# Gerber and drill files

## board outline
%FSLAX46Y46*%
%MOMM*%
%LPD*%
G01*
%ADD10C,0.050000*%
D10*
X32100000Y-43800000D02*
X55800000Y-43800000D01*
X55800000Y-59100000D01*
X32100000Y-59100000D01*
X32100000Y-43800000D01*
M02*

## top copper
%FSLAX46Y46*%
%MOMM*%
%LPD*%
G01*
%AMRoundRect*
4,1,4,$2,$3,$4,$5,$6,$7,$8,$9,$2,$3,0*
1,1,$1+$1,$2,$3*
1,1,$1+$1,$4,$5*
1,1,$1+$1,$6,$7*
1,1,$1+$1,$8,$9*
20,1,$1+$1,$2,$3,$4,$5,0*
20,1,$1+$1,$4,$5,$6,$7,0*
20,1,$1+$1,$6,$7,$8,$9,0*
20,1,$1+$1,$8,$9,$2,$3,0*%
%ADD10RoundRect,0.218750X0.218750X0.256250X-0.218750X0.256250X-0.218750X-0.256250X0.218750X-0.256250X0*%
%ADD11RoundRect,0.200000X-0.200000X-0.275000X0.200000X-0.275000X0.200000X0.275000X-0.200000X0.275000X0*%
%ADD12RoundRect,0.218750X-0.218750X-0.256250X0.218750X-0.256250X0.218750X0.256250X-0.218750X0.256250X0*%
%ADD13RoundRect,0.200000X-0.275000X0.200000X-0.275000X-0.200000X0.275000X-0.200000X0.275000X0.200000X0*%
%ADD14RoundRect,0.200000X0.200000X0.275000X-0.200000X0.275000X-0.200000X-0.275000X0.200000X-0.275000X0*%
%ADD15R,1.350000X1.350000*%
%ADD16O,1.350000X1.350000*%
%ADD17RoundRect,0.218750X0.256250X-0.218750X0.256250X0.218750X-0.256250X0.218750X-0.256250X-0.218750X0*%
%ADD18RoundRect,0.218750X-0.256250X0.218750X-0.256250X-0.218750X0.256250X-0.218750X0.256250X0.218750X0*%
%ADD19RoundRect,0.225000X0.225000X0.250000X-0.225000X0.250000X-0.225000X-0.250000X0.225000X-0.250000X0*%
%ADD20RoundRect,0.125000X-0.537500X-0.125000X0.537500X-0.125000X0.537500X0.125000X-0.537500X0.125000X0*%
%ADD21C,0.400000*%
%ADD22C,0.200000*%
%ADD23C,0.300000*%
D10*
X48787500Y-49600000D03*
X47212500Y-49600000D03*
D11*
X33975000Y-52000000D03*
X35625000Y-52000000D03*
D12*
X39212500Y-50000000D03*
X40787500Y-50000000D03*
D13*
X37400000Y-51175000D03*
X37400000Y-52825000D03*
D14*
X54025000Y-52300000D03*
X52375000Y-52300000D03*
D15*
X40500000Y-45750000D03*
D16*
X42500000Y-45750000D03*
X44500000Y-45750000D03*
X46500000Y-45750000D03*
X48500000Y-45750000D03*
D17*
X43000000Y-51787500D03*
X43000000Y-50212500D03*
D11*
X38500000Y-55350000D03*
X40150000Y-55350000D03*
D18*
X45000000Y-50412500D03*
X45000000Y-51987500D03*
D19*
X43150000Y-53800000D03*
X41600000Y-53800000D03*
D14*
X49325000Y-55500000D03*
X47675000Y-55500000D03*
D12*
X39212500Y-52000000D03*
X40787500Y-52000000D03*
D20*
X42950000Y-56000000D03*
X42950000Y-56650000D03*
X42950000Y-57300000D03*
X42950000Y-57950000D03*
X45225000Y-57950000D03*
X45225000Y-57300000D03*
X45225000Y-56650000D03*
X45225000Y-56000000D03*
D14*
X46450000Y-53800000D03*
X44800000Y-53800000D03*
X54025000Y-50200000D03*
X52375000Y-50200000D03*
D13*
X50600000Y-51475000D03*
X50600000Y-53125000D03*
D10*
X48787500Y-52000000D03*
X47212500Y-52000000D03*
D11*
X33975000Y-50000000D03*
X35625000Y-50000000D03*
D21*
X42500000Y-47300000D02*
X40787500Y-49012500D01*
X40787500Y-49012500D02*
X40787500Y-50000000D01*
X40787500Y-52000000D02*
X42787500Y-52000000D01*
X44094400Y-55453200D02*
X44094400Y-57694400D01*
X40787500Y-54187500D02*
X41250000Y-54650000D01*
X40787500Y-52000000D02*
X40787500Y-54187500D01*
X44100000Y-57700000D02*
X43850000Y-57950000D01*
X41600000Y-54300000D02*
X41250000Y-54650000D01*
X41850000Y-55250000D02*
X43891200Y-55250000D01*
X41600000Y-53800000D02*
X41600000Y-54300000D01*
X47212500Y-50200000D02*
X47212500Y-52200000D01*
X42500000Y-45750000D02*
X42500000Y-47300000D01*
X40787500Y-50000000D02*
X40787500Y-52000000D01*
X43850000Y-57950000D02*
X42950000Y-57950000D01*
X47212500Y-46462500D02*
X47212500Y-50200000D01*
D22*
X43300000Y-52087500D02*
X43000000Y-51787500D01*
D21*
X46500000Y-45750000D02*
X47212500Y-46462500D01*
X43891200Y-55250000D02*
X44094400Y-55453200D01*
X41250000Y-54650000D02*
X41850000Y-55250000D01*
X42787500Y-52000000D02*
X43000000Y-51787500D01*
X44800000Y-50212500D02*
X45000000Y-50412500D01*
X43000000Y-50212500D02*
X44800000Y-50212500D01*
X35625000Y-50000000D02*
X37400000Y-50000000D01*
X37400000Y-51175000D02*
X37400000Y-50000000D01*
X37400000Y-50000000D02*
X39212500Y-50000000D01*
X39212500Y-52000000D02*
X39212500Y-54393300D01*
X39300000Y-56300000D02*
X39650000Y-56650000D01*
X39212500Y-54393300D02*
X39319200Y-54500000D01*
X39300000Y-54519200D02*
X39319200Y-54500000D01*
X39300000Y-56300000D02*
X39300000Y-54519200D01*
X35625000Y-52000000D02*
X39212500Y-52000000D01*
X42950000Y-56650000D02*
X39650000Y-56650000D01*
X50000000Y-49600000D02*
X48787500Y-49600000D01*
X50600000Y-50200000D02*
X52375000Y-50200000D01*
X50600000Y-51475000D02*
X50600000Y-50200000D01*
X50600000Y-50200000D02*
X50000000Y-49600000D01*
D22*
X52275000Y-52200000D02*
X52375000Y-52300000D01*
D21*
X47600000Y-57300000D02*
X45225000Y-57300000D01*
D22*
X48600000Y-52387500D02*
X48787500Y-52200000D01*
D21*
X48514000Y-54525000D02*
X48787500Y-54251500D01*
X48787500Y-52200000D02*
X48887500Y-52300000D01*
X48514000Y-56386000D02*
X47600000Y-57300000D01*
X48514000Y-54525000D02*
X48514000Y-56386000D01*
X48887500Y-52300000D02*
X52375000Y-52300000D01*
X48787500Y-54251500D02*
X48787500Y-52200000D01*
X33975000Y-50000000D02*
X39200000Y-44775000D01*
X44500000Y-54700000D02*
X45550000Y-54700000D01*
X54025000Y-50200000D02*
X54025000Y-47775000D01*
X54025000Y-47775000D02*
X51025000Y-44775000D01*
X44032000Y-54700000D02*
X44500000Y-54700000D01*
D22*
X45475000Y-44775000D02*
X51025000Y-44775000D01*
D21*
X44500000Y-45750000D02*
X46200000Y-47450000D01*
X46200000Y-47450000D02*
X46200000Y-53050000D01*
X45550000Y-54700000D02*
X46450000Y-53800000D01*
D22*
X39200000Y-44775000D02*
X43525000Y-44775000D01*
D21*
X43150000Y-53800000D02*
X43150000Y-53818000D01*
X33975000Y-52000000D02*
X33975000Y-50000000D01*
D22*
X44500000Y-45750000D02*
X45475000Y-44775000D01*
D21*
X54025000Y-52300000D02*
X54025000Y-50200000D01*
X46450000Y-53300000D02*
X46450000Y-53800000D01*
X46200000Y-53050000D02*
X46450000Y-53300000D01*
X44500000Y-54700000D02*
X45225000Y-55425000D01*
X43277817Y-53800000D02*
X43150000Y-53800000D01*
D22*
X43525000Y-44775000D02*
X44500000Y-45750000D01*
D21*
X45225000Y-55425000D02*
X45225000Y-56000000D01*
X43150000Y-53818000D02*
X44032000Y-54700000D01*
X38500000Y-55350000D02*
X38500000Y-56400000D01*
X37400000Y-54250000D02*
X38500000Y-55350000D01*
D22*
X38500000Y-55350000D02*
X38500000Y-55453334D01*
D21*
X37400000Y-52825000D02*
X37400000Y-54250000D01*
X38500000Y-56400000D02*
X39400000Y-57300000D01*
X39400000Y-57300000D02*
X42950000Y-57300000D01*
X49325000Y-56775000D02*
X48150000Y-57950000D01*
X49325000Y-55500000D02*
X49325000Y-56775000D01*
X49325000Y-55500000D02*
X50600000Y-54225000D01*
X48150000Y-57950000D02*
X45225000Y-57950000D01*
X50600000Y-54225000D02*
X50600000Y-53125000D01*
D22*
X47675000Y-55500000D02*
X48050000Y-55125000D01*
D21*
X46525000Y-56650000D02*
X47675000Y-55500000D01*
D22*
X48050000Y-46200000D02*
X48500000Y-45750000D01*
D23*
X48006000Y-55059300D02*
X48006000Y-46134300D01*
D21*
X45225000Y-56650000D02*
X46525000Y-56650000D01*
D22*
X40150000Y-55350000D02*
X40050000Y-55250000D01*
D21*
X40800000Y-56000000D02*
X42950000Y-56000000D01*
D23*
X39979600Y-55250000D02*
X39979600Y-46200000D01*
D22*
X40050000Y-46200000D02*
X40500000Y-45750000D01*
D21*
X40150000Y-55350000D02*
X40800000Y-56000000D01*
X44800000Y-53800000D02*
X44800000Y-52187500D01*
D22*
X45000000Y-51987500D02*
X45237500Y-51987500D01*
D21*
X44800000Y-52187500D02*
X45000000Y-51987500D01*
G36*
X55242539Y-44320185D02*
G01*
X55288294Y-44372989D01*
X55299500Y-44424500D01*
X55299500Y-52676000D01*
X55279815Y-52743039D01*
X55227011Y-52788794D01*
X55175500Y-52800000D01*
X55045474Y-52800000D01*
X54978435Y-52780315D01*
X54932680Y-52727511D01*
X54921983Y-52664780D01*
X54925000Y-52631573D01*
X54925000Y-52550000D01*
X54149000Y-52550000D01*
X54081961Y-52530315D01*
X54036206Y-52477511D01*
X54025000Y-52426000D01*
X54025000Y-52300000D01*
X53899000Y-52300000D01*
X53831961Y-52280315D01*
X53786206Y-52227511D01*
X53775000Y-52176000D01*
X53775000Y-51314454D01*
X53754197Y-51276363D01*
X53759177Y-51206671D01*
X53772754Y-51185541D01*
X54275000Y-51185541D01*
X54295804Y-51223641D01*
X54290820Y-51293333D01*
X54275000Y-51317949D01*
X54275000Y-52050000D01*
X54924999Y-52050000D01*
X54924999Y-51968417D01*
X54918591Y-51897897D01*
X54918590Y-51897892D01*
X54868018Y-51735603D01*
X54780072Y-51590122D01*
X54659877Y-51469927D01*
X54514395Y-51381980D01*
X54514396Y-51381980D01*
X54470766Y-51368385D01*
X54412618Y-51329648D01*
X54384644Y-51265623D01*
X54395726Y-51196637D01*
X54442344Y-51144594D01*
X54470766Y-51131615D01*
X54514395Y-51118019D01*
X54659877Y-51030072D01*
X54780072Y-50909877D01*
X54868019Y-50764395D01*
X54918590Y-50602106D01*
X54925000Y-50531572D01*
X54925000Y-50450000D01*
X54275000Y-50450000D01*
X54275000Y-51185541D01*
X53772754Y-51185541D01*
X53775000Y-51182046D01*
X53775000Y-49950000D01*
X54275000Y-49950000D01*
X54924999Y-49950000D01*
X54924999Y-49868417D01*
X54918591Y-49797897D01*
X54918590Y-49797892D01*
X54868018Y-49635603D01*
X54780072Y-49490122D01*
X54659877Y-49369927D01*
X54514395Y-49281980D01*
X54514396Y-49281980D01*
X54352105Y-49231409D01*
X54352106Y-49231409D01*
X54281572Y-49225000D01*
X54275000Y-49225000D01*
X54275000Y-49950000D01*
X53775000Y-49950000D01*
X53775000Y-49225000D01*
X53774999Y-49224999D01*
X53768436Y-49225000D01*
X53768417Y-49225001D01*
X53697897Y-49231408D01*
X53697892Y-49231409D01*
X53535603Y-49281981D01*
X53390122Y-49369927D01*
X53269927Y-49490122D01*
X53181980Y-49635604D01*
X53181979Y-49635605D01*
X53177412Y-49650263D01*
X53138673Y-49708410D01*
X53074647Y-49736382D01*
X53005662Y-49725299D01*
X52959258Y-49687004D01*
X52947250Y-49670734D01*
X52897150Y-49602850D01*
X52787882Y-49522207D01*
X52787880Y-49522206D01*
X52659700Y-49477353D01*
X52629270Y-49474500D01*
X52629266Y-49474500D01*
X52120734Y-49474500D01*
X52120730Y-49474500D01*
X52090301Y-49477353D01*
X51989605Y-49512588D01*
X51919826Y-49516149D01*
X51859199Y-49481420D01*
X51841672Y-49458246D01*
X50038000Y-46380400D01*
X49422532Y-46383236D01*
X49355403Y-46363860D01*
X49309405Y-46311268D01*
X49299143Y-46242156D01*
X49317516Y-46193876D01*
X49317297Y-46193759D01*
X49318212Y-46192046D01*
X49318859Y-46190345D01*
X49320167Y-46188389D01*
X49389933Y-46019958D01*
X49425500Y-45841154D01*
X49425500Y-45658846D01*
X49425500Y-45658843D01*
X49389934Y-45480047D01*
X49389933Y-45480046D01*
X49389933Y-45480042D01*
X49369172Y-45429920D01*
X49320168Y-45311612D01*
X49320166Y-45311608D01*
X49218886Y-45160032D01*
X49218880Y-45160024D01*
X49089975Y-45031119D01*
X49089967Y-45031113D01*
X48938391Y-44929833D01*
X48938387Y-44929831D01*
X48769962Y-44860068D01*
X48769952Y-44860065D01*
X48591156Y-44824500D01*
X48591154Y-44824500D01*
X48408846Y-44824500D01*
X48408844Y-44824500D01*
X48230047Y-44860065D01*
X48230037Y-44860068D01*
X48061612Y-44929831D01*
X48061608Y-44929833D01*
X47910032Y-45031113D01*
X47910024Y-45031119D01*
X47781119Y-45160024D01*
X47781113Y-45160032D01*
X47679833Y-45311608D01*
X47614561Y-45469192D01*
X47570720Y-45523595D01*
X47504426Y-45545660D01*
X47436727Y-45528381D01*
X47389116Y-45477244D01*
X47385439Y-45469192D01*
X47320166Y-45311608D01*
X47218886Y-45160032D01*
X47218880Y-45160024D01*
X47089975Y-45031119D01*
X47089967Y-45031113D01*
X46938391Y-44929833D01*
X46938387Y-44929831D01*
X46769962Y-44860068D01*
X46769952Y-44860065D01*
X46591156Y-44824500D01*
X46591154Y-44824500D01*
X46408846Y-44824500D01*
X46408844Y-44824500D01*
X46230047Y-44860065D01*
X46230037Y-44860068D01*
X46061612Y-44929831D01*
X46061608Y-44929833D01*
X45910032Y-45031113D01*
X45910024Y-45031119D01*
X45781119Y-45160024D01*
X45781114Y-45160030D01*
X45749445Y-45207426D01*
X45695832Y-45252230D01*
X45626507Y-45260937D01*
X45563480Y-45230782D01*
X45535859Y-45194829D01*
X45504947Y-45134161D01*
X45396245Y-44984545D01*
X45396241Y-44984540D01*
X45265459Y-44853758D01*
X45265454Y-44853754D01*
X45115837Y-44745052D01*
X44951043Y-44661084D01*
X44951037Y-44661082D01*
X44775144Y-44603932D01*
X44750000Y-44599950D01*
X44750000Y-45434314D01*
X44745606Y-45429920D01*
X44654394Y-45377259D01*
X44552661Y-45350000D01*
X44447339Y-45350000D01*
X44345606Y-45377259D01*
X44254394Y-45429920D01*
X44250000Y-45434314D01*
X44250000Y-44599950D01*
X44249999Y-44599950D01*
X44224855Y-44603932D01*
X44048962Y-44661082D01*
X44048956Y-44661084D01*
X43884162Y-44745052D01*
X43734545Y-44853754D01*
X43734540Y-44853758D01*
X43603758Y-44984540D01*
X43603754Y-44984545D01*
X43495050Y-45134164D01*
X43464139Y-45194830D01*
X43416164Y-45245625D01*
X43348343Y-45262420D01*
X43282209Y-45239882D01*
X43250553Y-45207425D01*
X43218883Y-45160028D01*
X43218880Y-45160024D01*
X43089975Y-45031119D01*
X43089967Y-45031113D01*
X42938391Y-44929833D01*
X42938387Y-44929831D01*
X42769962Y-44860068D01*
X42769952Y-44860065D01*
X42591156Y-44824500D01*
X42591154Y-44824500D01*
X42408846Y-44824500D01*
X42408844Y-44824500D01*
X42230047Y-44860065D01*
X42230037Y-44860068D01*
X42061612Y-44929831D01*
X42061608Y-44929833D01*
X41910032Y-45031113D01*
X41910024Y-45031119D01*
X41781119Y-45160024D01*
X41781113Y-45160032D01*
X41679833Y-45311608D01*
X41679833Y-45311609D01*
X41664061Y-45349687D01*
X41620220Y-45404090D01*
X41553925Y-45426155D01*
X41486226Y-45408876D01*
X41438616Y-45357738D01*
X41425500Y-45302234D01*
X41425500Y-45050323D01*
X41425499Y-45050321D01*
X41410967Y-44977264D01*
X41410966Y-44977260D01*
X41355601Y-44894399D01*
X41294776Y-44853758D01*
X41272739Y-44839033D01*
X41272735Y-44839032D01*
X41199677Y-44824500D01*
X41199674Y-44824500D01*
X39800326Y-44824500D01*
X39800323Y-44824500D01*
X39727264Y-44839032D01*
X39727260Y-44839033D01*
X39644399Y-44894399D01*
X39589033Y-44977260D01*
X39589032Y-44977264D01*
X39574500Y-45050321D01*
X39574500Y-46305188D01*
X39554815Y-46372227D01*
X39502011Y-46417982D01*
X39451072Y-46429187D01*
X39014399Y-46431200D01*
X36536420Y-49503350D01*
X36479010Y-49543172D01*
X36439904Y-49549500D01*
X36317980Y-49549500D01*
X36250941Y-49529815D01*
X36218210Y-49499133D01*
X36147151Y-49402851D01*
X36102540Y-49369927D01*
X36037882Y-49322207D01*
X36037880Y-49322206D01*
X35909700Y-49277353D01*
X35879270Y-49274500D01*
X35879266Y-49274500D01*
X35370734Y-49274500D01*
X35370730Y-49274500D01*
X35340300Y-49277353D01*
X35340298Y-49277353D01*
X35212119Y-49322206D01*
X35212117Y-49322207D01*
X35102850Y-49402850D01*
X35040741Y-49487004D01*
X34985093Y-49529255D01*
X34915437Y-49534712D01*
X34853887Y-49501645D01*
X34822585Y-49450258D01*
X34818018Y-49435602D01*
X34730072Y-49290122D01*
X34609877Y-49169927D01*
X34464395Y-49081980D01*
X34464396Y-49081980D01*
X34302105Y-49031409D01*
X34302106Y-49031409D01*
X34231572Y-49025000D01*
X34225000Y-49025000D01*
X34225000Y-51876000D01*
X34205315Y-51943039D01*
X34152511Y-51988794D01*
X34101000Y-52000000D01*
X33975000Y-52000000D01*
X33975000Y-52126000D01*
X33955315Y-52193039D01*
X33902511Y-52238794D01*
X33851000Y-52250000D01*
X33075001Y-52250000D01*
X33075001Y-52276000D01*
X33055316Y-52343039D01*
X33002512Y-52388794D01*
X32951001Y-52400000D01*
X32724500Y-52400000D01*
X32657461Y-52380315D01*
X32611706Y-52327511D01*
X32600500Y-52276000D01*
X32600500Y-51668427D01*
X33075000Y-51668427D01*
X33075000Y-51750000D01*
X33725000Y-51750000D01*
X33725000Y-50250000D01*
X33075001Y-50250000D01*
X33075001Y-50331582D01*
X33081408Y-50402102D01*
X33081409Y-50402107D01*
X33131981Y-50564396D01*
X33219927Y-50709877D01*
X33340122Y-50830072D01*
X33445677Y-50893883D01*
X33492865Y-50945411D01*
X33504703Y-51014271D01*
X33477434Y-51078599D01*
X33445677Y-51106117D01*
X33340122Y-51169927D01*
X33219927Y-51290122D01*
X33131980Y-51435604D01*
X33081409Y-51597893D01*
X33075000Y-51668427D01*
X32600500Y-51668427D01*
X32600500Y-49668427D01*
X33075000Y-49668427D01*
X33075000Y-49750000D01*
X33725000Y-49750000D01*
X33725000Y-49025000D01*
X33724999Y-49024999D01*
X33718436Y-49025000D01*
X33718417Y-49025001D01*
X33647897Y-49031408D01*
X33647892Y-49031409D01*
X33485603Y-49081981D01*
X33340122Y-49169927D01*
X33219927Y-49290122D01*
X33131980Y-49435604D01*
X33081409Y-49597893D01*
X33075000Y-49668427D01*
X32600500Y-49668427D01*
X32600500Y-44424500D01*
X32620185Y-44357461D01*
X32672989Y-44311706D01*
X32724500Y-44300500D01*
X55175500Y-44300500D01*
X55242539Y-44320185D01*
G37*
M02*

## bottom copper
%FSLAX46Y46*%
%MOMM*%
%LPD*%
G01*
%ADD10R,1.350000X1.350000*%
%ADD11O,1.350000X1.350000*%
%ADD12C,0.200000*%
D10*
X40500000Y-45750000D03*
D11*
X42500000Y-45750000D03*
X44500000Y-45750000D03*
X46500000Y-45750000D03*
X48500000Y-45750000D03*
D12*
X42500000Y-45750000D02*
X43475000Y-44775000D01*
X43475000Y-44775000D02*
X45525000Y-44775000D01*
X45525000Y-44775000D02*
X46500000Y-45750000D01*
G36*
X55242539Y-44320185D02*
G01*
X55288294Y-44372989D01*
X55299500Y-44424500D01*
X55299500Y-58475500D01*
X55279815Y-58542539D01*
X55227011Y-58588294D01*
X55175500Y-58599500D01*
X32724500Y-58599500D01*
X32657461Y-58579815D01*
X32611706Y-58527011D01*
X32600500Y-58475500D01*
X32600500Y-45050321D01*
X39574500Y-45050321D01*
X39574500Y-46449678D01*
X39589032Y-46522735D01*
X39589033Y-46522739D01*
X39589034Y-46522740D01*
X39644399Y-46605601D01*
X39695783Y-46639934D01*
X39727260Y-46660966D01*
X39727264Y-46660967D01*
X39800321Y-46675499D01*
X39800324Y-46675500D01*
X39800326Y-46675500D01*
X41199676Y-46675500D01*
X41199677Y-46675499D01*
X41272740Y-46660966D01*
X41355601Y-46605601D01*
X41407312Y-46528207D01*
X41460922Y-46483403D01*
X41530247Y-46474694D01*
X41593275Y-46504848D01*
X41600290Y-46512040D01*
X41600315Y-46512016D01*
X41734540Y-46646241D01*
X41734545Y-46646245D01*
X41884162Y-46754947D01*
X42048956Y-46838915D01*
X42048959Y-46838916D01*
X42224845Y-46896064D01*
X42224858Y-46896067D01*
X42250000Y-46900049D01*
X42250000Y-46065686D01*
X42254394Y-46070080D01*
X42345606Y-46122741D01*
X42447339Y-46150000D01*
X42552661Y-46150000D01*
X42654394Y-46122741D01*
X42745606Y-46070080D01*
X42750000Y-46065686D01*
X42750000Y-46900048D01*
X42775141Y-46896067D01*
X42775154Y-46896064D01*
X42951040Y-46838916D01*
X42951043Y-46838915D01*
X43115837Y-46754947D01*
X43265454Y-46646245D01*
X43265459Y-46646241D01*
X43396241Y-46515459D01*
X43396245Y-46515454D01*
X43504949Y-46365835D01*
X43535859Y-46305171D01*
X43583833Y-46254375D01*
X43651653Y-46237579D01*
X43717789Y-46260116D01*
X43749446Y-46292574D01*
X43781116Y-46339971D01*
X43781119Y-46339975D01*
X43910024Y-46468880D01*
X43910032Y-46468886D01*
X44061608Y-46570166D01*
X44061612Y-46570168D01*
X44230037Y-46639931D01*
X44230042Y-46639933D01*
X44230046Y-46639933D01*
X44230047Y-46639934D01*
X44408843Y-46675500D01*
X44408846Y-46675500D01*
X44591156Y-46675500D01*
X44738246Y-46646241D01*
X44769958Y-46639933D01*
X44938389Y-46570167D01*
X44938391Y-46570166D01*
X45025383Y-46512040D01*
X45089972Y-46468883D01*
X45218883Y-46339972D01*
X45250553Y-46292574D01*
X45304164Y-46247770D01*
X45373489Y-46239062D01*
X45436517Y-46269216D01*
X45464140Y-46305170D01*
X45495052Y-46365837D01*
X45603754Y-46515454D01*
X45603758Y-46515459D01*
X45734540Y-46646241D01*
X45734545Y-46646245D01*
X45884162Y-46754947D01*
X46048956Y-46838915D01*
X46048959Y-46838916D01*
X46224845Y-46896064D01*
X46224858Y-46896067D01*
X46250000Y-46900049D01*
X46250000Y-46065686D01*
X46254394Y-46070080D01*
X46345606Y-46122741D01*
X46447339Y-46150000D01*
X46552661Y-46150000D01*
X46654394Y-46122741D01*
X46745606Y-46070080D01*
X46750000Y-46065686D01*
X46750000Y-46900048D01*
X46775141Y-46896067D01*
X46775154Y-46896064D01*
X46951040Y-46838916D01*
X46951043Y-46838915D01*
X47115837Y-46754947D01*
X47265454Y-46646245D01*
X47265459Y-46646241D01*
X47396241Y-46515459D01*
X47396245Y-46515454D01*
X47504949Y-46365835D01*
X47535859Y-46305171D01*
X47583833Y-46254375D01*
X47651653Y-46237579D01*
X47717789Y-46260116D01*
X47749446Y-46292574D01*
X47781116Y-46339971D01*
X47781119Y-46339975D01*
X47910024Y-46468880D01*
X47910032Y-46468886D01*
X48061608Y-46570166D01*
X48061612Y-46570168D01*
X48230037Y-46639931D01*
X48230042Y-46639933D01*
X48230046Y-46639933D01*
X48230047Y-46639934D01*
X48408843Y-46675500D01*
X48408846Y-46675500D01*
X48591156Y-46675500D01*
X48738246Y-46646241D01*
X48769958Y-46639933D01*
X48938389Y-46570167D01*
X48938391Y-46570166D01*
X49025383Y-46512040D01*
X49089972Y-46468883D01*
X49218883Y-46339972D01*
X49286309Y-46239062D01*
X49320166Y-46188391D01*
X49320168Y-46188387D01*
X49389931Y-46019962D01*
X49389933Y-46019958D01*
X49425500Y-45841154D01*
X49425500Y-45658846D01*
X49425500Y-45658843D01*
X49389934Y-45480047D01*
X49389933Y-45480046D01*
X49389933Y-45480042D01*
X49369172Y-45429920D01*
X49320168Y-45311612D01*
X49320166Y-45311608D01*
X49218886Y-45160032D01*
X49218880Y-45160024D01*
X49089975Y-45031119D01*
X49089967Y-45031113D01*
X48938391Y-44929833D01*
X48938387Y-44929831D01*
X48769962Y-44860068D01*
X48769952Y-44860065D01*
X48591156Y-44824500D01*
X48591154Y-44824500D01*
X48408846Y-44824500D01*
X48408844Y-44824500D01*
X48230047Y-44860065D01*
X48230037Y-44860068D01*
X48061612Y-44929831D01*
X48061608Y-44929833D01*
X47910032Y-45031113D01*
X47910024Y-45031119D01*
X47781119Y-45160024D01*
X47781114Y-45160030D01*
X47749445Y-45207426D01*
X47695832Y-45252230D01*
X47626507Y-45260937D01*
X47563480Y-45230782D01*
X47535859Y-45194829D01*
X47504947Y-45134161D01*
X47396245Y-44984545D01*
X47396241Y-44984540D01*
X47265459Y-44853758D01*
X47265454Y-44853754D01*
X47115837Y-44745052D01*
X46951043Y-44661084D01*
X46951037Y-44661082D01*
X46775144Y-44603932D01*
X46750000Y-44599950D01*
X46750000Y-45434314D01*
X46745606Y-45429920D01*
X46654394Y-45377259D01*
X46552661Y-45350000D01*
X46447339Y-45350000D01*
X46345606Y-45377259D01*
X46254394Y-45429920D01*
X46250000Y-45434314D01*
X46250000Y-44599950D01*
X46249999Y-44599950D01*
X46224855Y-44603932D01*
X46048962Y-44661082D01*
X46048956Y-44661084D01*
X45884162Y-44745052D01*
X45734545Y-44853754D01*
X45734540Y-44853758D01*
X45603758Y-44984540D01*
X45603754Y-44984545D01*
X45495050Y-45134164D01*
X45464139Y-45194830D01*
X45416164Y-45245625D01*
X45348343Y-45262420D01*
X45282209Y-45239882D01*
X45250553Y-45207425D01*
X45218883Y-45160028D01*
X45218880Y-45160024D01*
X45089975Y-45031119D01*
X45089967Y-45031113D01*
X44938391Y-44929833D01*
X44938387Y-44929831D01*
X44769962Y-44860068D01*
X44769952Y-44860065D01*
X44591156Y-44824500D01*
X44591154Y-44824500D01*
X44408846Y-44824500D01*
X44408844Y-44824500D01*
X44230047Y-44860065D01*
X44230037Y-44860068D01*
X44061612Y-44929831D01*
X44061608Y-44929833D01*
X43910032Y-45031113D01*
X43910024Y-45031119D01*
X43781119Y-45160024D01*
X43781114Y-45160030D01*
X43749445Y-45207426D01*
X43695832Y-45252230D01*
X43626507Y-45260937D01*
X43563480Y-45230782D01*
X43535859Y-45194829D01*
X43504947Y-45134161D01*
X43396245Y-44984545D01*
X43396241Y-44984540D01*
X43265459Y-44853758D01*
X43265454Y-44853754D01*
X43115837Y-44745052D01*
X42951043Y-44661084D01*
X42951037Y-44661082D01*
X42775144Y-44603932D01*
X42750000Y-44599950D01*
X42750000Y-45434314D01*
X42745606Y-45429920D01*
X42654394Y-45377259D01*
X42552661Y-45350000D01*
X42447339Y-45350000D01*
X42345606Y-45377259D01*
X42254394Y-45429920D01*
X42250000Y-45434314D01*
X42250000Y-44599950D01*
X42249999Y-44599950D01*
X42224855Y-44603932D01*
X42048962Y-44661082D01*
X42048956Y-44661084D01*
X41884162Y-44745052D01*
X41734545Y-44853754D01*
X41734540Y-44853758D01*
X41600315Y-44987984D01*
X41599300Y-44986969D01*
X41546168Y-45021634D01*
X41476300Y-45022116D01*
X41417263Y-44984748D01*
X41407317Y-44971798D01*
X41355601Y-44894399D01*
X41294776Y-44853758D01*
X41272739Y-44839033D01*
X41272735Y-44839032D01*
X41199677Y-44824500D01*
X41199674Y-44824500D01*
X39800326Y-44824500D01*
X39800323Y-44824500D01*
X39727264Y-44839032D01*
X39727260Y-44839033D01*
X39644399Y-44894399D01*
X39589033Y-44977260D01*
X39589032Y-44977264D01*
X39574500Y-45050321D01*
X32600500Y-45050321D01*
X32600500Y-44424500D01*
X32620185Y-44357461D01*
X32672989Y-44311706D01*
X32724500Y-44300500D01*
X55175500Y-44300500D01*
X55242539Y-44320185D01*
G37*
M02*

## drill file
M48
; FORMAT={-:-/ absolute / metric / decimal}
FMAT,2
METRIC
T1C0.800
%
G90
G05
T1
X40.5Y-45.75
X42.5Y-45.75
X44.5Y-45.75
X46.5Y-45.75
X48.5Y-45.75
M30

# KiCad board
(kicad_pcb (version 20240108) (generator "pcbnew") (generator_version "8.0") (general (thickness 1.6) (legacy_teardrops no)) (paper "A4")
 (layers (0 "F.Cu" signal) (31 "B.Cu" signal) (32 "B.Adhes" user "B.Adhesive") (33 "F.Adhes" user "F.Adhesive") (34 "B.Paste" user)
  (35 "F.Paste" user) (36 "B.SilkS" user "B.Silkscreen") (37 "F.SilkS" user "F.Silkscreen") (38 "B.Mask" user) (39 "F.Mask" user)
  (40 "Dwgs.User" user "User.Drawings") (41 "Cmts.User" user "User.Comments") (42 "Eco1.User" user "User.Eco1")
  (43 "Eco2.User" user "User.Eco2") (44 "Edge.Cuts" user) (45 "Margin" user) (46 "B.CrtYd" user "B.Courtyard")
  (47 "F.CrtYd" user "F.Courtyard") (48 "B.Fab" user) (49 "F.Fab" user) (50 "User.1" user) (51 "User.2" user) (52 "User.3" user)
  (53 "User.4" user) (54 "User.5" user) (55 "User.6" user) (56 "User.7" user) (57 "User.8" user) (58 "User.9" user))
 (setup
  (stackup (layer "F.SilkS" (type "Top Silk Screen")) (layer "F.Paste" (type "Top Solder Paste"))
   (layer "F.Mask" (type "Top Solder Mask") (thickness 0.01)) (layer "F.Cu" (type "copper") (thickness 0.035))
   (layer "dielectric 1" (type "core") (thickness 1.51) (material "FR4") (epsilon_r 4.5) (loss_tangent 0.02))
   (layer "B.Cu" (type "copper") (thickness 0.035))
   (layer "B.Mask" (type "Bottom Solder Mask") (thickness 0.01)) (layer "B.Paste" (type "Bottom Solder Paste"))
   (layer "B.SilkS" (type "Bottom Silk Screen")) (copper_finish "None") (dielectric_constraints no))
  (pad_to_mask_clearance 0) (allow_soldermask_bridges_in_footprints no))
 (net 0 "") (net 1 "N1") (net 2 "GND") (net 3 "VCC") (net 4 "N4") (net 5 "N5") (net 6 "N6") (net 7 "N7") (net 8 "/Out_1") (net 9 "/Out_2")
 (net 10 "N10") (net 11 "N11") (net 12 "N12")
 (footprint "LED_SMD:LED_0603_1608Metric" (layer "F.Cu") (at 48 49.6 180)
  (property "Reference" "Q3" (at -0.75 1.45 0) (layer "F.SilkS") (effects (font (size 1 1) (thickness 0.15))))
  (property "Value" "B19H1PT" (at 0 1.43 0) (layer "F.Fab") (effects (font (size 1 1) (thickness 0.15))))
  (pad "1" smd roundrect (at -0.7875 0 180) (size 0.875 0.95) (layers "F.Cu" "F.Paste" "F.Mask") (roundrect_rratio 0.25) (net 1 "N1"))
  (pad "2" smd roundrect (at 0.7875 0 180) (size 0.875 0.95) (layers "F.Cu" "F.Paste" "F.Mask") (roundrect_rratio 0.25) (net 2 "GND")))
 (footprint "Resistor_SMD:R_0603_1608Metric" (layer "F.Cu") (at 34.8 52)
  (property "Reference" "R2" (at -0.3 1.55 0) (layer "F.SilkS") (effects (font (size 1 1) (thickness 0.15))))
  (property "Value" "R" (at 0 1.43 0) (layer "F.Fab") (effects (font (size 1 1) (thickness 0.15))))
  (pad "1" smd roundrect (at -0.825 0) (size 0.8 0.95) (layers "F.Cu" "F.Paste" "F.Mask") (roundrect_rratio 0.25) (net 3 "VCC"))
  (pad "2" smd roundrect (at 0.825 0) (size 0.8 0.95) (layers "F.Cu" "F.Paste" "F.Mask") (roundrect_rratio 0.25) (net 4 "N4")))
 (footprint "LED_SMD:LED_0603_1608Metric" (layer "F.Cu") (at 40 50)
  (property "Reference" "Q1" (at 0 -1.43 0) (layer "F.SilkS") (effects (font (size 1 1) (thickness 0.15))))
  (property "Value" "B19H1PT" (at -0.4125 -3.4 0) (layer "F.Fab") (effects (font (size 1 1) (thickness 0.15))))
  (pad "1" smd roundrect (at -0.7875 0) (size 0.875 0.95) (layers "F.Cu" "F.Paste" "F.Mask") (roundrect_rratio 0.25) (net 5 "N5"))
  (pad "2" smd roundrect (at 0.7875 0) (size 0.875 0.95) (layers "F.Cu" "F.Paste" "F.Mask") (roundrect_rratio 0.25) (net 2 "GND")))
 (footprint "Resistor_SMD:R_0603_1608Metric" (layer "F.Cu") (at 37.4 52 -90)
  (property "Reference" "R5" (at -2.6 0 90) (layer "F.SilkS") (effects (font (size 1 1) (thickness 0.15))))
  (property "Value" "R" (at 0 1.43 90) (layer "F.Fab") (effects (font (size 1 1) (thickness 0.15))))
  (pad "1" smd roundrect (at -0.825 0 270) (size 0.8 0.95) (layers "F.Cu" "F.Paste" "F.Mask") (roundrect_rratio 0.25) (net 5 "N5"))
  (pad "2" smd roundrect (at 0.825 0 270) (size 0.8 0.95) (layers "F.Cu" "F.Paste" "F.Mask") (roundrect_rratio 0.25) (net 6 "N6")))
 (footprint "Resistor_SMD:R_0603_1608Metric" (layer "F.Cu") (at 53.2 52.3 180)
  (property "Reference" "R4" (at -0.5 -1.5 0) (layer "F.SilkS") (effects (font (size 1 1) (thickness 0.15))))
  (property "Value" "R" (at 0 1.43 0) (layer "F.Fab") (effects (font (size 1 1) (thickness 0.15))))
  (pad "1" smd roundrect (at -0.825 0 180) (size 0.8 0.95) (layers "F.Cu" "F.Paste" "F.Mask") (roundrect_rratio 0.25) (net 3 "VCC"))
  (pad "2" smd roundrect (at 0.825 0 180) (size 0.8 0.95) (layers "F.Cu" "F.Paste" "F.Mask") (roundrect_rratio 0.25) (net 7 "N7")))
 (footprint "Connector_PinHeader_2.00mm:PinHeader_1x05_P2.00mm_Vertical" (layer "F.Cu") (at 40.5 45.75 90)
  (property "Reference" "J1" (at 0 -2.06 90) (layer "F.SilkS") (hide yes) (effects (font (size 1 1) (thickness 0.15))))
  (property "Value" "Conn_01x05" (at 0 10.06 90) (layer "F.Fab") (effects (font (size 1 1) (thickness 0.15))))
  (pad "1" thru_hole rect (at 0 0 90) (size 1.35 1.35) (drill 0.8) (layers "*.Cu" "*.Mask") (remove_unused_layers no) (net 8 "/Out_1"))
  (pad "2" thru_hole oval (at 0 2 90) (size 1.35 1.35) (drill 0.8) (layers "*.Cu" "*.Mask") (remove_unused_layers no) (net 2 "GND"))
  (pad "3" thru_hole oval (at 0 4 90) (size 1.35 1.35) (drill 0.8) (layers "*.Cu" "*.Mask") (remove_unused_layers no) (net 3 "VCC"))
  (pad "4" thru_hole oval (at 0 6 90) (size 1.35 1.35) (drill 0.8) (layers "*.Cu" "*.Mask") (remove_unused_layers no) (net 2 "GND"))
  (pad "5" thru_hole oval (at 0 8 90) (size 1.35 1.35) (drill 0.8) (layers "*.Cu" "*.Mask") (remove_unused_layers no) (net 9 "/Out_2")))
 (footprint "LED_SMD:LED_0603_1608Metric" (layer "F.Cu") (at 43 51 90)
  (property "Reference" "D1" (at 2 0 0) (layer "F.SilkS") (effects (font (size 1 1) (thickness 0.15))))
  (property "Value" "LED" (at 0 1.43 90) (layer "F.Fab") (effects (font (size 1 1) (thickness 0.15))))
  (pad "1" smd roundrect (at -0.7875 0 90) (size 0.875 0.95) (layers "F.Cu" "F.Paste" "F.Mask") (roundrect_rratio 0.25) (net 2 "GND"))
  (pad "2" smd roundrect (at 0.7875 0 90) (size 0.875 0.95) (layers "F.Cu" "F.Paste" "F.Mask") (roundrect_rratio 0.25) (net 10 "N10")))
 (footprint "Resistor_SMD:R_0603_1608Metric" (layer "F.Cu") (at 39.325 55.35)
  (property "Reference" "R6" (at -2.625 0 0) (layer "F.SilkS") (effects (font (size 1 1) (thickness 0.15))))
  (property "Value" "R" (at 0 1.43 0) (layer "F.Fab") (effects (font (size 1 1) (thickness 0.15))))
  (pad "1" smd roundrect (at -0.825 0) (size 0.8 0.95) (layers "F.Cu" "F.Paste" "F.Mask") (roundrect_rratio 0.25) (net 6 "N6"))
  (pad "2" smd roundrect (at 0.825 0) (size 0.8 0.95) (layers "F.Cu" "F.Paste" "F.Mask") (roundrect_rratio 0.25) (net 8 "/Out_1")))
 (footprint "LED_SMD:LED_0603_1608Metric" (layer "F.Cu") (at 45 51.2 -90)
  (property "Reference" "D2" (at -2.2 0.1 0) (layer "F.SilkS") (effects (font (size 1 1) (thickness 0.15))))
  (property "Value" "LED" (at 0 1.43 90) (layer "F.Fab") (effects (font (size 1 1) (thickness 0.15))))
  (pad "1" smd roundrect (at -0.7875 0 270) (size 0.875 0.95) (layers "F.Cu" "F.Paste" "F.Mask") (roundrect_rratio 0.25) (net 10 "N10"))
  (pad "2" smd roundrect (at 0.7875 0 270) (size 0.875 0.95) (layers "F.Cu" "F.Paste" "F.Mask") (roundrect_rratio 0.25) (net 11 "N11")))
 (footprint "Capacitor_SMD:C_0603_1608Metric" (layer "F.Cu") (at 42.375 53.8 180)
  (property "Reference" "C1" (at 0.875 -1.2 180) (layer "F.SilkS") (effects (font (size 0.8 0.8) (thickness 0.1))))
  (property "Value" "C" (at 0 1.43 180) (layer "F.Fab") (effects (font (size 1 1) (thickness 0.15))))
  (pad "1" smd roundrect (at -0.775 0 180) (size 0.9 0.95) (layers "F.Cu" "F.Paste" "F.Mask") (roundrect_rratio 0.25) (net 3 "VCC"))
  (pad "2" smd roundrect (at 0.775 0 180) (size 0.9 0.95) (layers "F.Cu" "F.Paste" "F.Mask") (roundrect_rratio 0.25) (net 2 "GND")))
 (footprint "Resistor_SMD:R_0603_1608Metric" (layer "F.Cu") (at 48.5 55.5 180)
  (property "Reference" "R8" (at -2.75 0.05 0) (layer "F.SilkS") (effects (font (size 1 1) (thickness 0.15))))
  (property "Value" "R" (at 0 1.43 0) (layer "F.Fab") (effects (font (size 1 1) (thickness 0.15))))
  (pad "1" smd roundrect (at -0.825 0 180) (size 0.8 0.95) (layers "F.Cu" "F.Paste" "F.Mask") (roundrect_rratio 0.25) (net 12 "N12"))
  (pad "2" smd roundrect (at 0.825 0 180) (size 0.8 0.95) (layers "F.Cu" "F.Paste" "F.Mask") (roundrect_rratio 0.25) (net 9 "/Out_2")))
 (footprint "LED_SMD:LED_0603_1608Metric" (layer "F.Cu") (at 40 52)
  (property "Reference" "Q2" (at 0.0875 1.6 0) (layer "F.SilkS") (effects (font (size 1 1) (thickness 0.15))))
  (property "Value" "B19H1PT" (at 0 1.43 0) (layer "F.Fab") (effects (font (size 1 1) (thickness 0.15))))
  (pad "1" smd roundrect (at -0.7875 0) (size 0.875 0.95) (layers "F.Cu" "F.Paste" "F.Mask") (roundrect_rratio 0.25) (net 4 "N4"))
  (pad "2" smd roundrect (at 0.7875 0) (size 0.875 0.95) (layers "F.Cu" "F.Paste" "F.Mask") (roundrect_rratio 0.25) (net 2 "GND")))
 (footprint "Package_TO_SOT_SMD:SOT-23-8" (layer "F.Cu") (at 44.0875 56.975)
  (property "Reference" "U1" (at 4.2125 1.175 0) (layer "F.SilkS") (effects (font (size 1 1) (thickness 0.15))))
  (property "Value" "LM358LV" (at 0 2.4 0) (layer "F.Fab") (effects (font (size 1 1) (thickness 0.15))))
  (pad "1" smd roundrect (at -1.1375 -0.975) (size 1.325 0.5) (layers "F.Cu" "F.Paste" "F.Mask") (roundrect_rratio 0.25) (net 8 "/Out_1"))
  (pad "2" smd roundrect (at -1.1375 -0.325) (size 1.325 0.5) (layers "F.Cu" "F.Paste" "F.Mask") (roundrect_rratio 0.25) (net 4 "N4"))
  (pad "3" smd roundrect (at -1.1375 0.325) (size 1.325 0.5) (layers "F.Cu" "F.Paste" "F.Mask") (roundrect_rratio 0.25) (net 6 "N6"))
  (pad "4" smd roundrect (at -1.1375 0.975) (size 1.325 0.5) (layers "F.Cu" "F.Paste" "F.Mask") (roundrect_rratio 0.25) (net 2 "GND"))
  (pad "5" smd roundrect (at 1.1375 0.975) (size 1.325 0.5) (layers "F.Cu" "F.Paste" "F.Mask") (roundrect_rratio 0.25) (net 12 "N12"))
  (pad "6" smd roundrect (at 1.1375 0.325) (size 1.325 0.5) (layers "F.Cu" "F.Paste" "F.Mask") (roundrect_rratio 0.25) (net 7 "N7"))
  (pad "7" smd roundrect (at 1.1375 -0.325) (size 1.325 0.5) (layers "F.Cu" "F.Paste" "F.Mask") (roundrect_rratio 0.25) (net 9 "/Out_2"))
  (pad "8" smd roundrect (at 1.1375 -0.975) (size 1.325 0.5) (layers "F.Cu" "F.Paste" "F.Mask") (roundrect_rratio 0.25) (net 3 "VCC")))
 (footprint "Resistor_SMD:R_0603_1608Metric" (layer "F.Cu") (at 45.625 53.8 180)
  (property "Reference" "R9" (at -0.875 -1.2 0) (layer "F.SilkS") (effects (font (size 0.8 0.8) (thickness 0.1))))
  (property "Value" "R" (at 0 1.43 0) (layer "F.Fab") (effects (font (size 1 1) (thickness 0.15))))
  (pad "1" smd roundrect (at -0.825 0 180) (size 0.8 0.95) (layers "F.Cu" "F.Paste" "F.Mask") (roundrect_rratio 0.25) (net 3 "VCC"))
  (pad "2" smd roundrect (at 0.825 0 180) (size 0.8 0.95) (layers "F.Cu" "F.Paste" "F.Mask") (roundrect_rratio 0.25) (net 11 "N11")))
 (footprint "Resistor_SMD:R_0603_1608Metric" (layer "F.Cu") (at 53.2 50.2 180)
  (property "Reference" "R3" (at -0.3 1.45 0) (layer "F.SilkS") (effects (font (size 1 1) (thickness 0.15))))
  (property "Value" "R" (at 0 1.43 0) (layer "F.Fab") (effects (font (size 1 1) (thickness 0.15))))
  (pad "1" smd roundrect (at -0.825 0 180) (size 0.8 0.95) (layers "F.Cu" "F.Paste" "F.Mask") (roundrect_rratio 0.25) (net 3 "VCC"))
  (pad "2" smd roundrect (at 0.825 0 180) (size 0.8 0.95) (layers "F.Cu" "F.Paste" "F.Mask") (roundrect_rratio 0.25) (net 1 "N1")))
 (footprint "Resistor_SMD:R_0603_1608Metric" (layer "F.Cu") (at 50.6 52.3 -90)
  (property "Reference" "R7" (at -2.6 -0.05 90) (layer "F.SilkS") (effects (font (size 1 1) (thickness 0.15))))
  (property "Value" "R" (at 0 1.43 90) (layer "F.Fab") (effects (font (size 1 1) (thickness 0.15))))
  (pad "1" smd roundrect (at -0.825 0 270) (size 0.8 0.95) (layers "F.Cu" "F.Paste" "F.Mask") (roundrect_rratio 0.25) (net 1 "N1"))
  (pad "2" smd roundrect (at 0.825 0 270) (size 0.8 0.95) (layers "F.Cu" "F.Paste" "F.Mask") (roundrect_rratio 0.25) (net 12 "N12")))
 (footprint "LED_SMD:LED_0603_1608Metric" (layer "F.Cu") (at 48 52 180)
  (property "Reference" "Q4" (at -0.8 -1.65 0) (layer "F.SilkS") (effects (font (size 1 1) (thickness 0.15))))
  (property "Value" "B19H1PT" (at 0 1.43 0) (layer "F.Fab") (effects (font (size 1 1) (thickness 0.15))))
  (pad "1" smd roundrect (at -0.7875 0 180) (size 0.875 0.95) (layers "F.Cu" "F.Paste" "F.Mask") (roundrect_rratio 0.25) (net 7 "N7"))
  (pad "2" smd roundrect (at 0.7875 0 180) (size 0.875 0.95) (layers "F.Cu" "F.Paste" "F.Mask") (roundrect_rratio 0.25) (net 2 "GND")))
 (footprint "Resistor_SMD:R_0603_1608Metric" (layer "F.Cu") (at 34.8 50)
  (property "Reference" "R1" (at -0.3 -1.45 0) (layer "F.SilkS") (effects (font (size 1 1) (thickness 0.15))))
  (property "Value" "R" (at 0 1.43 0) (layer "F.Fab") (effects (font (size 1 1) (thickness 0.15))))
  (pad "1" smd roundrect (at -0.825 0) (size 0.8 0.95) (layers "F.Cu" "F.Paste" "F.Mask") (roundrect_rratio 0.25) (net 3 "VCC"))
  (pad "2" smd roundrect (at 0.825 0) (size 0.8 0.95) (layers "F.Cu" "F.Paste" "F.Mask") (roundrect_rratio 0.25) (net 5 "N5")))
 (gr_rect (start 32.1 43.8) (end 55.8 59.1) (stroke (width 0.05) (type default)) (fill none) (layer "Edge.Cuts"))
 (segment (start 42.5 47.3) (end 40.7875 49.0125) (width 0.4) (layer "F.Cu") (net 2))
 (segment (start 40.7875 49.0125) (end 40.7875 50) (width 0.4) (layer "F.Cu") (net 2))
 (segment (start 40.7875 52) (end 42.7875 52) (width 0.4) (layer "F.Cu") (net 2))
 (segment (start 44.0944 55.4532) (end 44.0944 57.6944) (width 0.4) (layer "F.Cu") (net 2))
 (segment (start 40.7875 54.1875) (end 41.25 54.65) (width 0.4) (layer "F.Cu") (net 2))
 (segment (start 40.7875 52) (end 40.7875 54.1875) (width 0.4) (layer "F.Cu") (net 2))
 (segment (start 44.1 57.7) (end 43.85 57.95) (width 0.4) (layer "F.Cu") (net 2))
 (segment (start 41.6 54.3) (end 41.25 54.65) (width 0.4) (layer "F.Cu") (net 2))
 (segment (start 41.85 55.25) (end 43.8912 55.25) (width 0.4) (layer "F.Cu") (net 2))
 (segment (start 41.6 53.8) (end 41.6 54.3) (width 0.4) (layer "F.Cu") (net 2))
 (segment (start 47.2125 50.2) (end 47.2125 52.2) (width 0.4) (layer "F.Cu") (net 2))
 (segment (start 42.5 45.75) (end 42.5 47.3) (width 0.4) (layer "F.Cu") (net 2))
 (segment (start 40.7875 50) (end 40.7875 52) (width 0.4) (layer "F.Cu") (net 2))
 (segment (start 43.85 57.95) (end 42.95 57.95) (width 0.4) (layer "F.Cu") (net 2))
 (segment (start 47.2125 46.4625) (end 47.2125 50.2) (width 0.4) (layer "F.Cu") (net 2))
 (segment (start 43.3 52.0875) (end 43 51.7875) (width 0.2) (layer "F.Cu") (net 2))
 (segment (start 46.5 45.75) (end 47.2125 46.4625) (width 0.4) (layer "F.Cu") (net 2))
 (segment (start 43.8912 55.25) (end 44.0944 55.4532) (width 0.4) (layer "F.Cu") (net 2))
 (segment (start 41.25 54.65) (end 41.85 55.25) (width 0.4) (layer "F.Cu") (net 2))
 (segment (start 42.7875 52) (end 43 51.7875) (width 0.4) (layer "F.Cu") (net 2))
 (segment (start 42.5 45.75) (end 43.475 44.775) (width 0.2) (layer "B.Cu") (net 2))
 (segment (start 43.475 44.775) (end 45.525 44.775) (width 0.2) (layer "B.Cu") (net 2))
 (segment (start 45.525 44.775) (end 46.5 45.75) (width 0.2) (layer "B.Cu") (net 2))
 (segment (start 44.8 50.2125) (end 45 50.4125) (width 0.4) (layer "F.Cu") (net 10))
 (segment (start 43 50.2125) (end 44.8 50.2125) (width 0.4) (layer "F.Cu") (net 10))
 (segment (start 35.625 50) (end 37.4 50) (width 0.4) (layer "F.Cu") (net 5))
 (segment (start 37.4 51.175) (end 37.4 50) (width 0.4) (layer "F.Cu") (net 5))
 (segment (start 37.4 50) (end 39.2125 50) (width 0.4) (layer "F.Cu") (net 5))
 (segment (start 39.2125 52) (end 39.2125 54.3933) (width 0.4) (layer "F.Cu") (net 4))
 (segment (start 39.3 56.3) (end 39.65 56.65) (width 0.4) (layer "F.Cu") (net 4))
 (segment (start 39.2125 54.3933) (end 39.3192 54.5) (width 0.4) (layer "F.Cu") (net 4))
 (segment (start 39.3 54.5192) (end 39.3192 54.5) (width 0.4) (layer "F.Cu") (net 4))
 (segment (start 39.3 56.3) (end 39.3 54.5192) (width 0.4) (layer "F.Cu") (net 4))
 (segment (start 35.625 52) (end 39.2125 52) (width 0.4) (layer "F.Cu") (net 4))
 (segment (start 42.95 56.65) (end 39.65 56.65) (width 0.4) (layer "F.Cu") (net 4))
 (segment (start 50 49.6) (end 48.7875 49.6) (width 0.4) (layer "F.Cu") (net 1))
 (segment (start 50.6 50.2) (end 52.375 50.2) (width 0.4) (layer "F.Cu") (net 1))
 (segment (start 50.6 51.475) (end 50.6 50.2) (width 0.4) (layer "F.Cu") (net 1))
 (segment (start 50.6 50.2) (end 50 49.6) (width 0.4) (layer "F.Cu") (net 1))
 (segment (start 52.275 52.2) (end 52.375 52.3) (width 0.2) (layer "F.Cu") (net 7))
 (segment (start 47.6 57.3) (end 45.225 57.3) (width 0.4) (layer "F.Cu") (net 7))
 (segment (start 48.6 52.3875) (end 48.7875 52.2) (width 0.2) (layer "F.Cu") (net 7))
 (segment (start 48.514 54.525) (end 48.7875 54.2515) (width 0.4) (layer "F.Cu") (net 7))
 (segment (start 48.7875 52.2) (end 48.8875 52.3) (width 0.4) (layer "F.Cu") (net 7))
 (segment (start 48.514 56.386) (end 47.6 57.3) (width 0.4) (layer "F.Cu") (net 7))
 (segment (start 48.514 54.525) (end 48.514 56.386) (width 0.4) (layer "F.Cu") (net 7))
 (segment (start 48.8875 52.3) (end 52.375 52.3) (width 0.4) (layer "F.Cu") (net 7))
 (segment (start 48.7875 54.2515) (end 48.7875 52.2) (width 0.4) (layer "F.Cu") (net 7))
 (segment (start 33.975 50) (end 39.2 44.775) (width 0.4) (layer "F.Cu") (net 3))
 (segment (start 44.5 54.7) (end 45.55 54.7) (width 0.4) (layer "F.Cu") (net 3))
 (segment (start 54.025 50.2) (end 54.025 47.775) (width 0.4) (layer "F.Cu") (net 3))
 (segment (start 54.025 47.775) (end 51.025 44.775) (width 0.4) (layer "F.Cu") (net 3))
 (segment (start 44.032 54.7) (end 44.5 54.7) (width 0.4) (layer "F.Cu") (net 3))
 (segment (start 45.475 44.775) (end 51.025 44.775) (width 0.2) (layer "F.Cu") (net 3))
 (segment (start 44.5 45.75) (end 46.2 47.45) (width 0.4) (layer "F.Cu") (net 3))
 (segment (start 46.2 47.45) (end 46.2 53.05) (width 0.4) (layer "F.Cu") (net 3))
 (segment (start 45.55 54.7) (end 46.45 53.8) (width 0.4) (layer "F.Cu") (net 3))
 (segment (start 39.2 44.775) (end 43.525 44.775) (width 0.2) (layer "F.Cu") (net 3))
 (segment (start 43.15 53.8) (end 43.15 53.818) (width 0.4) (layer "F.Cu") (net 3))
 (segment (start 33.975 52) (end 33.975 50) (width 0.4) (layer "F.Cu") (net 3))
 (segment (start 44.5 45.75) (end 45.475 44.775) (width 0.2) (layer "F.Cu") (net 3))
 (segment (start 54.025 52.3) (end 54.025 50.2) (width 0.4) (layer "F.Cu") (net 3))
 (segment (start 46.45 53.3) (end 46.45 53.8) (width 0.4) (layer "F.Cu") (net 3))
 (segment (start 46.2 53.05) (end 46.45 53.3) (width 0.4) (layer "F.Cu") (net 3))
 (segment (start 44.5 54.7) (end 45.225 55.425) (width 0.4) (layer "F.Cu") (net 3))
 (segment (start 43.277817 53.8) (end 43.15 53.8) (width 0.4) (layer "F.Cu") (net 3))
 (segment (start 43.525 44.775) (end 44.5 45.75) (width 0.2) (layer "F.Cu") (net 3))
 (segment (start 45.225 55.425) (end 45.225 56) (width 0.4) (layer "F.Cu") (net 3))
 (segment (start 43.15 53.818) (end 44.032 54.7) (width 0.4) (layer "F.Cu") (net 3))
 (segment (start 38.5 55.35) (end 38.5 56.4) (width 0.4) (layer "F.Cu") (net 6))
 (segment (start 37.4 54.25) (end 38.5 55.35) (width 0.4) (layer "F.Cu") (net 6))
 (segment (start 38.5 55.35) (end 38.5 55.453334) (width 0.2) (layer "F.Cu") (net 6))
 (segment (start 37.4 52.825) (end 37.4 54.25) (width 0.4) (layer "F.Cu") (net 6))
 (segment (start 38.5 56.4) (end 39.4 57.3) (width 0.4) (layer "F.Cu") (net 6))
 (segment (start 39.4 57.3) (end 42.95 57.3) (width 0.4) (layer "F.Cu") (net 6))
 (segment (start 49.325 56.775) (end 48.15 57.95) (width 0.4) (layer "F.Cu") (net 12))
 (segment (start 49.325 55.5) (end 49.325 56.775) (width 0.4) (layer "F.Cu") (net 12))
 (segment (start 49.325 55.5) (end 50.6 54.225) (width 0.4) (layer "F.Cu") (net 12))
 (segment (start 48.15 57.95) (end 45.225 57.95) (width 0.4) (layer "F.Cu") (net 12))
 (segment (start 50.6 54.225) (end 50.6 53.125) (width 0.4) (layer "F.Cu") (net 12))
 (segment (start 47.675 55.5) (end 48.05 55.125) (width 0.2) (layer "F.Cu") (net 9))
 (segment (start 46.525 56.65) (end 47.675 55.5) (width 0.4) (layer "F.Cu") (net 9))
 (segment (start 48.05 46.2) (end 48.5 45.75) (width 0.2) (layer "F.Cu") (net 9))
 (segment (start 48.006 55.0593) (end 48.006 46.1343) (width 0.3) (layer "F.Cu") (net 9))
 (segment (start 45.225 56.65) (end 46.525 56.65) (width 0.4) (layer "F.Cu") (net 9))
 (segment (start 40.15 55.35) (end 40.05 55.25) (width 0.2) (layer "F.Cu") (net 8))
 (segment (start 40.8 56) (end 42.95 56) (width 0.4) (layer "F.Cu") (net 8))
 (segment (start 39.9796 55.25) (end 39.9796 46.2) (width 0.3) (layer "F.Cu") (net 8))
 (segment (start 40.05 46.2) (end 40.5 45.75) (width 0.2) (layer "F.Cu") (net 8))
 (segment (start 40.15 55.35) (end 40.8 56) (width 0.4) (layer "F.Cu") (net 8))
 (segment (start 44.8 53.8) (end 44.8 52.1875) (width 0.4) (layer "F.Cu") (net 11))
 (segment (start 45 51.9875) (end 45.2375 51.9875) (width 0.2) (layer "F.Cu") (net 11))
 (segment (start 44.8 52.1875) (end 45 51.9875) (width 0.4) (layer "F.Cu") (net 11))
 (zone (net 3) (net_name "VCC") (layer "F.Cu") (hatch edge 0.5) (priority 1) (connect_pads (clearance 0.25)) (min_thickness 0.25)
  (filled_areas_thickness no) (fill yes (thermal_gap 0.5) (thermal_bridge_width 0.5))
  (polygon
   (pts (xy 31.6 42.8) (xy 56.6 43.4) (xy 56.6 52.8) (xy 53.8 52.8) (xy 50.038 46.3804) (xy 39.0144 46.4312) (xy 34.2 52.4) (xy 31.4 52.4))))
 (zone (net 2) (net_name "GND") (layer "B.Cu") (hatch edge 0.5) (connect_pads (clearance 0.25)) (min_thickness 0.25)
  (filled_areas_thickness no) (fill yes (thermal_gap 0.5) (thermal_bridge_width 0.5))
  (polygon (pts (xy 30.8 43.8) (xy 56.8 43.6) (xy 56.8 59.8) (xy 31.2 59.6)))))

